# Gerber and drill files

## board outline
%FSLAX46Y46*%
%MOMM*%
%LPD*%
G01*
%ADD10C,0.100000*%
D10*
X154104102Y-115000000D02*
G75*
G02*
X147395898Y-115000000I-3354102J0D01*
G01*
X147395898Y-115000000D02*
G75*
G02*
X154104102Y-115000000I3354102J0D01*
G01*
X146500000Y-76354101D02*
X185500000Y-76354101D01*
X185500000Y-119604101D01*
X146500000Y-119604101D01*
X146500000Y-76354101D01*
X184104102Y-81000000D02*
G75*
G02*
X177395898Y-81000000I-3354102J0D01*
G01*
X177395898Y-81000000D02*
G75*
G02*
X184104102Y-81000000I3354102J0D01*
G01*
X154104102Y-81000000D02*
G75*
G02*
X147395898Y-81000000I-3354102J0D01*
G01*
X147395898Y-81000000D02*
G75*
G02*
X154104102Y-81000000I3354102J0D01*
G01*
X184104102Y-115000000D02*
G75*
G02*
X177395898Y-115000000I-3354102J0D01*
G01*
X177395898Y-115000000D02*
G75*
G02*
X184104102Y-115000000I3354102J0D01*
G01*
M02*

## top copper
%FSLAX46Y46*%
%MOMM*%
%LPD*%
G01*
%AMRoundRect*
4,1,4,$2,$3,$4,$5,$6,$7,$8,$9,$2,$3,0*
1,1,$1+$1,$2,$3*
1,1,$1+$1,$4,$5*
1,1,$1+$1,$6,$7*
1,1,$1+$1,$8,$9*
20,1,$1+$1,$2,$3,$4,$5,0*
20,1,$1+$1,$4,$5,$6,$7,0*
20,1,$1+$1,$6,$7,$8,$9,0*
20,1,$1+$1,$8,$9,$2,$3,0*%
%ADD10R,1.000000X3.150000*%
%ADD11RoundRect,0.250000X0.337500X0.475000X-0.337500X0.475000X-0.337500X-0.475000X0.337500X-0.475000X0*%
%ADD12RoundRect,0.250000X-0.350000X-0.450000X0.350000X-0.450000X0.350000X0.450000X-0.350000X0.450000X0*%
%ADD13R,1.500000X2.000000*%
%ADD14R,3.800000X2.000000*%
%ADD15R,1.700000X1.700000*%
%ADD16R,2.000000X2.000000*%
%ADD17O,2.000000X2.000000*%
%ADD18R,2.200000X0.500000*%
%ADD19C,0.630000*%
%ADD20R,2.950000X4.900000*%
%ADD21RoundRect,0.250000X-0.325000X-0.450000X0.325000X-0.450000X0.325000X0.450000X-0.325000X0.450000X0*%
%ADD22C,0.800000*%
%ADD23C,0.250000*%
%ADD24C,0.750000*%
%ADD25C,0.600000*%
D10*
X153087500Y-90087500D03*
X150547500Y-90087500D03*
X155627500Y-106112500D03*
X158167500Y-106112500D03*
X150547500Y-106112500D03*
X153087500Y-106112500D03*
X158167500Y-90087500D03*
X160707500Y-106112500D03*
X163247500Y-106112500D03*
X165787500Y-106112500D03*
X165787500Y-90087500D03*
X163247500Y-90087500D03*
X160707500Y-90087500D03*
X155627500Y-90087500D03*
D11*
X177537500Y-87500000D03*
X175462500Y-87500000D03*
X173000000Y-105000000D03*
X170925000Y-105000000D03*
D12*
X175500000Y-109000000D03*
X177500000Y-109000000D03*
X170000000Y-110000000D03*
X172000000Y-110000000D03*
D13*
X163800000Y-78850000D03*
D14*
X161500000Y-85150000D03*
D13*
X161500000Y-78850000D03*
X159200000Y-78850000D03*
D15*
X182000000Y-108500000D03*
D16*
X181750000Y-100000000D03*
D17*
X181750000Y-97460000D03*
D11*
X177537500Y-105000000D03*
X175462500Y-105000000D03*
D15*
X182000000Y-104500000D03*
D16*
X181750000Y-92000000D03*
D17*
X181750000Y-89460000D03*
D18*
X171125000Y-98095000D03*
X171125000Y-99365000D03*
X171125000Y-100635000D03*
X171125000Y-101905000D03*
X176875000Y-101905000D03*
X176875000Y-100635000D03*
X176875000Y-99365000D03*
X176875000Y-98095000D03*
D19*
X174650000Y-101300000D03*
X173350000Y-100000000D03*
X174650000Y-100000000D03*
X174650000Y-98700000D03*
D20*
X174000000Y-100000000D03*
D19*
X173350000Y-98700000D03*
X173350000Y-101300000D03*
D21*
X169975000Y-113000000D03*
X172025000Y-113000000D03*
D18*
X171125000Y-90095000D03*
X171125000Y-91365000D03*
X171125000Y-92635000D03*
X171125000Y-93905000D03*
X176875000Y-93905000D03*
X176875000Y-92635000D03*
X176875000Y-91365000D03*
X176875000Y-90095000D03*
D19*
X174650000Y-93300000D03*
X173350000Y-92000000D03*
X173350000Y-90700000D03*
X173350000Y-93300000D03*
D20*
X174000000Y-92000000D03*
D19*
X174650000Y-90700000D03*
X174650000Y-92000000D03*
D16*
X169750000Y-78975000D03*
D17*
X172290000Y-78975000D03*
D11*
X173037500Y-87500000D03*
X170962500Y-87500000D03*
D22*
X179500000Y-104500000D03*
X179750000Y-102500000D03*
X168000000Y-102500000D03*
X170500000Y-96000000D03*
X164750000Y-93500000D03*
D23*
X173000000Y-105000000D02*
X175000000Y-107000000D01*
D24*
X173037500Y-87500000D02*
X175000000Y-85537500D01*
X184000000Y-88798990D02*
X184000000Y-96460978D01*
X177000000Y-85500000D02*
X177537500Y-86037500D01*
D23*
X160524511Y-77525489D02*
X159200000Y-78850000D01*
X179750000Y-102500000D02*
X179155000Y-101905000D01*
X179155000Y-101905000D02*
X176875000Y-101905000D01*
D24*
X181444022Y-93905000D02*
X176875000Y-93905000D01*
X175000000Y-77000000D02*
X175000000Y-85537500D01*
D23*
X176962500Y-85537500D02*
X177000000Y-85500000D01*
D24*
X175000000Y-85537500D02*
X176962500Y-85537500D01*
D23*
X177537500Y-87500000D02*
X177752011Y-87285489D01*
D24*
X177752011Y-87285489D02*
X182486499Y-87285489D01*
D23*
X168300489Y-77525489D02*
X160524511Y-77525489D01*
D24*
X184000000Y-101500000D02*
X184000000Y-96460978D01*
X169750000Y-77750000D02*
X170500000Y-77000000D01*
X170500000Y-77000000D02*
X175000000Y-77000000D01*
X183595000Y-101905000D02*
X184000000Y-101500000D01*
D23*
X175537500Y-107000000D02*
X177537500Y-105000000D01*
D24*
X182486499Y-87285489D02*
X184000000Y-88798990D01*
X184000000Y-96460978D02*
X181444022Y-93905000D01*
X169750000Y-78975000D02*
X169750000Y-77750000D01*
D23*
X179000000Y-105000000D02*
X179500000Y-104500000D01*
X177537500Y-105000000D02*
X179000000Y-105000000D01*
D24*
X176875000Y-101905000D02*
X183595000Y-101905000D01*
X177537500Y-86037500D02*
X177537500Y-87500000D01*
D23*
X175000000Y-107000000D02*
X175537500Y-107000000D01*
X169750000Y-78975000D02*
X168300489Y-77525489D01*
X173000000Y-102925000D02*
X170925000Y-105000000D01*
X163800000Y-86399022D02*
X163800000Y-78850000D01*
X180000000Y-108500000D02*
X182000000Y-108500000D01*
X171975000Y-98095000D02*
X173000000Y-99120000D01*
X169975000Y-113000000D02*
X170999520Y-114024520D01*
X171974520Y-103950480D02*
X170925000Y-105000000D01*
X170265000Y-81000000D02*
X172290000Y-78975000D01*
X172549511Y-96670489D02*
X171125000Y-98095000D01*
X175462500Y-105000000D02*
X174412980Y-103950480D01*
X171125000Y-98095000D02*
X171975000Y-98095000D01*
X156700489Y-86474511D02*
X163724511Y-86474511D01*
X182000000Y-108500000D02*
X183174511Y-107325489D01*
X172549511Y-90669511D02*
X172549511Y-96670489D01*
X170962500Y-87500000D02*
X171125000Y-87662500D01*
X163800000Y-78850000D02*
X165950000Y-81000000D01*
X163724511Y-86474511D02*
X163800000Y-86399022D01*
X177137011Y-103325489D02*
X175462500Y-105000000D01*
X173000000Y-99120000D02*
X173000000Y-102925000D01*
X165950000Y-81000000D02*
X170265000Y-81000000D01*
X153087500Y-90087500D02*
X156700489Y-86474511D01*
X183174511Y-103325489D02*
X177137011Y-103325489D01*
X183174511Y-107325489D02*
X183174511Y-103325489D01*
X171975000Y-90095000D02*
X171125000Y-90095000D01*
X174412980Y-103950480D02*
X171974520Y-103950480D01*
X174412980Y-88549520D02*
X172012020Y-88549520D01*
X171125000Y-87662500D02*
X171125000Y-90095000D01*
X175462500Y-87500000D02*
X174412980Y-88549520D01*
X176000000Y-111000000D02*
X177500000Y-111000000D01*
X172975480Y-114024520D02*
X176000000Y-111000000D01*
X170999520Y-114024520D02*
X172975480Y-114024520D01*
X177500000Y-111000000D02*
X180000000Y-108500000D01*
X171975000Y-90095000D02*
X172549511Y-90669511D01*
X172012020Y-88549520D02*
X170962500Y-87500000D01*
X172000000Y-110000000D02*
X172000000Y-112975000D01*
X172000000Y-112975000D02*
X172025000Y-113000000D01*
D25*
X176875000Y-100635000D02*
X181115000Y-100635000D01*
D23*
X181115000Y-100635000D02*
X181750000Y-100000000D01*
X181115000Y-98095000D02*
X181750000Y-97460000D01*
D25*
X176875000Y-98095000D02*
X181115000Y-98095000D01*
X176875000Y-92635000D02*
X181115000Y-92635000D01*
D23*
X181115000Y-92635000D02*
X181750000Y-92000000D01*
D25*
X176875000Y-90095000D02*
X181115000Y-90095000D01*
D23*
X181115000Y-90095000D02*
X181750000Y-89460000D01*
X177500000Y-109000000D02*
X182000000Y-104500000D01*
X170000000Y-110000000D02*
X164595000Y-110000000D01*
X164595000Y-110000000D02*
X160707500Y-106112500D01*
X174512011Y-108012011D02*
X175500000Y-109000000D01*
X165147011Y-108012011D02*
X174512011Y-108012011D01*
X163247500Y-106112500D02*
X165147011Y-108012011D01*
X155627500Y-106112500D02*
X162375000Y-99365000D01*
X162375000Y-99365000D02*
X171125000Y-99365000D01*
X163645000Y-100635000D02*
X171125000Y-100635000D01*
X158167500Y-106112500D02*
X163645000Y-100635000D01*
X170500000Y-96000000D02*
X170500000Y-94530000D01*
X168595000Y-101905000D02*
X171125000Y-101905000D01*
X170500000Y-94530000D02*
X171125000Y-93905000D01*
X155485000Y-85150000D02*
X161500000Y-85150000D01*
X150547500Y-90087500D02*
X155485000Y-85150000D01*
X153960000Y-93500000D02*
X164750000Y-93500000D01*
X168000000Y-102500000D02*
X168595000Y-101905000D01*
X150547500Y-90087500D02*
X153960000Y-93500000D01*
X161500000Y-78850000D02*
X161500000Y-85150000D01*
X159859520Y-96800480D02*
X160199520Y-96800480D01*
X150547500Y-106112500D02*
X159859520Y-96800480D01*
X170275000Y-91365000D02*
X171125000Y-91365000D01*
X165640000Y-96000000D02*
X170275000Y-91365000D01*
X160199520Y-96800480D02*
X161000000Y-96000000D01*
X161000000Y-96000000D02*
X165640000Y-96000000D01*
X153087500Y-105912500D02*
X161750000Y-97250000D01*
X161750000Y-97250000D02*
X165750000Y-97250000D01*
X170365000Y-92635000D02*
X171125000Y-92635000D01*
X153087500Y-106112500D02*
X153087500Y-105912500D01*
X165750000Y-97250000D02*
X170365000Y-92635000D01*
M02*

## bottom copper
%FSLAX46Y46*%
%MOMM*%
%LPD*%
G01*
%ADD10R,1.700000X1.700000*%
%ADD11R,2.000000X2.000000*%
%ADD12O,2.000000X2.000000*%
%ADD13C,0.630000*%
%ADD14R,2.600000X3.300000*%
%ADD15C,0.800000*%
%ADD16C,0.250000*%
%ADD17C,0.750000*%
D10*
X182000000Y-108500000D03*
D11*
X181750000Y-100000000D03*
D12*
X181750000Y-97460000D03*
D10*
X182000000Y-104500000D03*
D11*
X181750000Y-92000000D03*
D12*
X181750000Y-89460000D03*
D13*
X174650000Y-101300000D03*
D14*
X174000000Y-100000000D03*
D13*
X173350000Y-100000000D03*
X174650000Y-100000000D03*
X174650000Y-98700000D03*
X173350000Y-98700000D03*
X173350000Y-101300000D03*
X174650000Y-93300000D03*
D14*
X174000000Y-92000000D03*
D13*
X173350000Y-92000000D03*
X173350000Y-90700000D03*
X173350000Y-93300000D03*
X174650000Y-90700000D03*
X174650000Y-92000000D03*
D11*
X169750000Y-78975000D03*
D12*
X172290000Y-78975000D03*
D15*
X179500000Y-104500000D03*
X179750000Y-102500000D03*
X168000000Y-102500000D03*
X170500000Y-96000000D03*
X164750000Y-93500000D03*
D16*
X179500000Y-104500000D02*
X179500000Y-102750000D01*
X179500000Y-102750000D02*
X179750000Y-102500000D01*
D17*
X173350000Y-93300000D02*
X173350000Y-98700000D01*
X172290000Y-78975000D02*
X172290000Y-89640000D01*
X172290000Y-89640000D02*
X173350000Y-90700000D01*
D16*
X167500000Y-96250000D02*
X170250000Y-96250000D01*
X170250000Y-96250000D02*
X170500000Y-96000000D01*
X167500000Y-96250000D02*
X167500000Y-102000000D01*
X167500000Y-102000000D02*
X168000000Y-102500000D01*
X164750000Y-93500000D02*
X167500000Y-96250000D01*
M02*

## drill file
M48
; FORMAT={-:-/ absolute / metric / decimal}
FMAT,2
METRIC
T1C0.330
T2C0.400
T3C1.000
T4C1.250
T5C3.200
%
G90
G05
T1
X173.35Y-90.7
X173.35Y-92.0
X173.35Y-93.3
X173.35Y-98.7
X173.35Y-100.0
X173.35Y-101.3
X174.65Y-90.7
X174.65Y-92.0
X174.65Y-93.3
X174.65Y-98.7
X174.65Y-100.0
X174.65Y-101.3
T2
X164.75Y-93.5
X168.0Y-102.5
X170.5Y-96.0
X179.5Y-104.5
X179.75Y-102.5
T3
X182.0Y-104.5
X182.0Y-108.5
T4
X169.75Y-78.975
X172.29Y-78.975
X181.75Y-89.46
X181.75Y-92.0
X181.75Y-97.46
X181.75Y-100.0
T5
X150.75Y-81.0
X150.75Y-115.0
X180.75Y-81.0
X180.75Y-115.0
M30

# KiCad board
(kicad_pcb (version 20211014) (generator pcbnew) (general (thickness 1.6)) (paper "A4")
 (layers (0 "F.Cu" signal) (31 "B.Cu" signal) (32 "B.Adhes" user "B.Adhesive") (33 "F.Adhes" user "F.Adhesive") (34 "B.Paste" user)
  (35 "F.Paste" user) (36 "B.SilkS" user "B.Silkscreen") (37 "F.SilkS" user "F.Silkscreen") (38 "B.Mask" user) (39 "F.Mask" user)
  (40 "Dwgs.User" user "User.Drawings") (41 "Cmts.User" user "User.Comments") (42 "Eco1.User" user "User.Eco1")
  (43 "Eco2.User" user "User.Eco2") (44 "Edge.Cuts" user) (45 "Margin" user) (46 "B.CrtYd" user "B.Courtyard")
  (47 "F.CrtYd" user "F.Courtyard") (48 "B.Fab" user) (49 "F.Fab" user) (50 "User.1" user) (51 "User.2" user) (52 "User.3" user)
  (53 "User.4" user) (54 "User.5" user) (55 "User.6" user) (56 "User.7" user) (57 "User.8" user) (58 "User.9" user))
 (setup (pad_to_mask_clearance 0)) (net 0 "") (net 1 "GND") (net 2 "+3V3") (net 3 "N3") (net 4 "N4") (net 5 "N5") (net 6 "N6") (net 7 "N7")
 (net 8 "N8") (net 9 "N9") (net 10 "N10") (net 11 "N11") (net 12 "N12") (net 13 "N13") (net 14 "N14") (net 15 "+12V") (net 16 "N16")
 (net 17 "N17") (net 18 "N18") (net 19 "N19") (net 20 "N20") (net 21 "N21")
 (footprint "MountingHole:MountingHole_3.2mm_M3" (layer "F.Cu") (at 180.75 115)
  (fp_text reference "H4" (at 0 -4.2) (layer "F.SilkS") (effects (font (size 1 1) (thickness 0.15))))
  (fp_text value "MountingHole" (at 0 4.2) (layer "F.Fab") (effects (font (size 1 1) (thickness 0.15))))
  (pad "" np_thru_hole circle (at 0 0) (size 3.2 3.2) (drill 3.2) (layers *.Cu *.Mask)))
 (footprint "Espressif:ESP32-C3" (layer "F.Cu") (at 159.9675 97.5125 90)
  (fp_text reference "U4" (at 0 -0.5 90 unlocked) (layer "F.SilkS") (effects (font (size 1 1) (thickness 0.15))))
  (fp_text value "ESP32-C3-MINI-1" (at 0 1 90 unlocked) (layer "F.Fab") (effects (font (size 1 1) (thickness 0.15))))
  (pad "1" smd rect (at 7.425 -6.88 90) (size 3.15 1) (layers "F.Cu" "F.Paste" "F.Mask") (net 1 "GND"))
  (pad "3" smd rect (at 7.425 -9.42 90) (size 3.15 1) (layers "F.Cu" "F.Paste" "F.Mask") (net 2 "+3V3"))
  (pad "5" smd rect (at -8.6 -4.34 90) (size 3.15 1) (layers "F.Cu" "F.Paste" "F.Mask") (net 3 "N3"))
  (pad "6" smd rect (at -8.6 -1.8 90) (size 3.15 1) (layers "F.Cu" "F.Paste" "F.Mask") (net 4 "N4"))
  (pad "12" smd rect (at -8.6 -9.42 90) (size 3.15 1) (layers "F.Cu" "F.Paste" "F.Mask") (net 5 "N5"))
  (pad "13" smd rect (at -8.6 -6.88 90) (size 3.15 1) (layers "F.Cu" "F.Paste" "F.Mask") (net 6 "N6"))
  (pad "16" smd rect (at 7.425 -1.8 90) (size 3.15 1) (layers "F.Cu" "F.Paste" "F.Mask") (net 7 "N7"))
  (pad "18" smd rect (at -8.6 0.74 90) (size 3.15 1) (layers "F.Cu" "F.Paste" "F.Mask") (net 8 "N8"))
  (pad "19" smd rect (at -8.6 3.28 90) (size 3.15 1) (layers "F.Cu" "F.Paste" "F.Mask") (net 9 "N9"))
  (pad "20" smd rect (at -8.6 5.82 90) (size 3.15 1) (layers "F.Cu" "F.Paste" "F.Mask") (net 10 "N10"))
  (pad "21" smd rect (at 7.425 5.82 90) (size 3.15 1) (layers "F.Cu" "F.Paste" "F.Mask") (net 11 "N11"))
  (pad "22" smd rect (at 7.425 3.28 90) (size 3.15 1) (layers "F.Cu" "F.Paste" "F.Mask") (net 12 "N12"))
  (pad "23" smd rect (at 7.425 0.74 90) (size 3.15 1) (layers "F.Cu" "F.Paste" "F.Mask") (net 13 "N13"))
  (pad "35" smd rect (at 7.425 -4.34 90) (size 3.15 1) (layers "F.Cu" "F.Paste" "F.Mask") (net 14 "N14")))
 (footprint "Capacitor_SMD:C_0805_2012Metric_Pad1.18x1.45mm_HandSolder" (layer "F.Cu") (at 176.5 87.5 180)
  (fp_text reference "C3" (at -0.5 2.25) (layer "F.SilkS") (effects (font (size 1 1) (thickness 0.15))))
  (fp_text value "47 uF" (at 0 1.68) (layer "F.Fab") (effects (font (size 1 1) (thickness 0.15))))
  (pad "1" smd roundrect (at -1.0375 0 180) (size 1.175 1.45) (layers "F.Cu" "F.Paste" "F.Mask") (roundrect_rratio 0.2127659574)
   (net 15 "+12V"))
  (pad "2" smd roundrect (at 1.0375 0 180) (size 1.175 1.45) (layers "F.Cu" "F.Paste" "F.Mask") (roundrect_rratio 0.2127659574)
   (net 1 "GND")))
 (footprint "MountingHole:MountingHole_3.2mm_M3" (layer "F.Cu") (at 180.75 81)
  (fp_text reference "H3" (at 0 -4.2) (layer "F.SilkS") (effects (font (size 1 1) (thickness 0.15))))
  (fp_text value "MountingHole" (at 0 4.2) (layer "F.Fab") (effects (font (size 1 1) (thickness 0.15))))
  (pad "" np_thru_hole circle (at 0 0) (size 3.2 3.2) (drill 3.2) (layers *.Cu *.Mask)))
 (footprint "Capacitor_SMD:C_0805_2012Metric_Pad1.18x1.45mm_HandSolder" (layer "F.Cu") (at 171.9625 105 180)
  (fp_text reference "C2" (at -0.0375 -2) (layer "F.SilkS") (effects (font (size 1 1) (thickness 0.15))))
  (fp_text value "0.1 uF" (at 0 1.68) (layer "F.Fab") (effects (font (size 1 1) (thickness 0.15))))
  (pad "1" smd roundrect (at -1.0375 0 180) (size 1.175 1.45) (layers "F.Cu" "F.Paste" "F.Mask") (roundrect_rratio 0.2127659574)
   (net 15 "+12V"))
  (pad "2" smd roundrect (at 1.0375 0 180) (size 1.175 1.45) (layers "F.Cu" "F.Paste" "F.Mask") (roundrect_rratio 0.2127659574)
   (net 1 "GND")))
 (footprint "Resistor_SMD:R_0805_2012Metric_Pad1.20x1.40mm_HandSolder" (layer "F.Cu") (at 176.5 109)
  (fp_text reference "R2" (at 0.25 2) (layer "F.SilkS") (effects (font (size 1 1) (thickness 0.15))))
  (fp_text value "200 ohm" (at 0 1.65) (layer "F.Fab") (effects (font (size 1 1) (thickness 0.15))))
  (pad "1" smd roundrect (at -1 0) (size 1.2 1.4) (layers "F.Cu" "F.Paste" "F.Mask") (roundrect_rratio 0.2083333333) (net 9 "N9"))
  (pad "2" smd roundrect (at 1 0) (size 1.2 1.4) (layers "F.Cu" "F.Paste" "F.Mask") (roundrect_rratio 0.2083333333) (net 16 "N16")))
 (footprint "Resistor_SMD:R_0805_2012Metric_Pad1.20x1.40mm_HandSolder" (layer "F.Cu") (at 171 110)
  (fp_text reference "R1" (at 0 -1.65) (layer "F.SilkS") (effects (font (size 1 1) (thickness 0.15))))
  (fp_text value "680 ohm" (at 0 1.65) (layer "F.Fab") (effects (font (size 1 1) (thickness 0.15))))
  (pad "1" smd roundrect (at -1 0) (size 1.2 1.4) (layers "F.Cu" "F.Paste" "F.Mask") (roundrect_rratio 0.2083333333) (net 8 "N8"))
  (pad "2" smd roundrect (at 1 0) (size 1.2 1.4) (layers "F.Cu" "F.Paste" "F.Mask") (roundrect_rratio 0.2083333333) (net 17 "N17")))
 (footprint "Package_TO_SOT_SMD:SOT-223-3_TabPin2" (layer "F.Cu") (at 161.5 82 -90)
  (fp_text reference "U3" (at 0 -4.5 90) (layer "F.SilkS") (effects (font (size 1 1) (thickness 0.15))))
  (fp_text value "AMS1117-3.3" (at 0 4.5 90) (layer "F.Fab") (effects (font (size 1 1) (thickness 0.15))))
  (pad "1" smd rect (at -3.15 -2.3 270) (size 2 1.5) (layers "F.Cu" "F.Paste" "F.Mask") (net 1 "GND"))
  (pad "2" smd rect (at 3.15 0 270) (size 2 3.8) (layers "F.Cu" "F.Paste" "F.Mask") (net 2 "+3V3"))
  (pad "2" smd rect (at -3.15 0 270) (size 2 1.5) (layers "F.Cu" "F.Paste" "F.Mask") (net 2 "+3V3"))
  (pad "3" smd rect (at -3.15 2.3 270) (size 2 1.5) (layers "F.Cu" "F.Paste" "F.Mask") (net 15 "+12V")))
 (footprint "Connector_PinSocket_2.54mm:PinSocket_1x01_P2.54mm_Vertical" (layer "F.Cu") (at 182 108.5 180)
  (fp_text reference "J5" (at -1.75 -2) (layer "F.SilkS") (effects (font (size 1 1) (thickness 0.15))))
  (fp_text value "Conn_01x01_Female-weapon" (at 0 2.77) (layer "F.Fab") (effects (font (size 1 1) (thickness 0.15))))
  (pad "1" thru_hole rect (at 0 0 180) (size 1.7 1.7) (drill 1) (layers *.Cu *.Mask) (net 1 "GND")))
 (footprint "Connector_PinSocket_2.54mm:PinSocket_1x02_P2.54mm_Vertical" (layer "F.Cu") (at 181.75 100 180)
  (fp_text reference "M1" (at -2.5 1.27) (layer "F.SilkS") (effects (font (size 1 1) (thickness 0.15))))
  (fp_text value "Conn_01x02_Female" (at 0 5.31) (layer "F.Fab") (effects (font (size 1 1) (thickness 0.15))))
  (pad "1" thru_hole rect (at 0 0 180) (size 2 2) (drill 1.25) (layers *.Cu *.Mask) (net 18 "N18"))
  (pad "2" thru_hole oval (at 0 2.54 180) (size 2 2) (drill 1.25) (layers *.Cu *.Mask) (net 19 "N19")))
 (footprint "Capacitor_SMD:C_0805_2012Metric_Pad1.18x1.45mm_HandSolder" (layer "F.Cu") (at 176.5 105 180)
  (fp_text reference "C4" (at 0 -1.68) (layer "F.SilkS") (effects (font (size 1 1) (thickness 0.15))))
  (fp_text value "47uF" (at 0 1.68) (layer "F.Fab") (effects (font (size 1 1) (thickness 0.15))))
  (pad "1" smd roundrect (at -1.0375 0 180) (size 1.175 1.45) (layers "F.Cu" "F.Paste" "F.Mask") (roundrect_rratio 0.2127659574)
   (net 15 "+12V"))
  (pad "2" smd roundrect (at 1.0375 0 180) (size 1.175 1.45) (layers "F.Cu" "F.Paste" "F.Mask") (roundrect_rratio 0.2127659574)
   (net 1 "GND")))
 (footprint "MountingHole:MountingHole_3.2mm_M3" (layer "F.Cu") (at 150.75 115)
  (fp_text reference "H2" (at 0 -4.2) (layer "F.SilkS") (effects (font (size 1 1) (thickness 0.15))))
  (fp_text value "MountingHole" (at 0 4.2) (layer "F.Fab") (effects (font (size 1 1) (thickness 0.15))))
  (pad "" np_thru_hole circle (at 0 0) (size 3.2 3.2) (drill 3.2) (layers *.Cu *.Mask)))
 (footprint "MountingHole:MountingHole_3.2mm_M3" (layer "F.Cu") (at 150.75 81)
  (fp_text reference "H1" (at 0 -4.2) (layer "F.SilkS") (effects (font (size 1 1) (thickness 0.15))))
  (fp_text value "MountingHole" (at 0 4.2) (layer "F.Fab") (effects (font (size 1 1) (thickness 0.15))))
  (pad "" np_thru_hole circle (at 0 0) (size 3.2 3.2) (drill 3.2) (layers *.Cu *.Mask)))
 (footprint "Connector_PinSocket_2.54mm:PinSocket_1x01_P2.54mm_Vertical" (layer "F.Cu") (at 182 104.5)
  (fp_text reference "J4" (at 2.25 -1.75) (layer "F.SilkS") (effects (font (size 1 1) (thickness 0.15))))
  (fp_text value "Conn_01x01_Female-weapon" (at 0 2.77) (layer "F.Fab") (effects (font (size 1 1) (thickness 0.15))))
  (pad "1" thru_hole rect (at 0 0) (size 1.7 1.7) (drill 1) (layers *.Cu *.Mask) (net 16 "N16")))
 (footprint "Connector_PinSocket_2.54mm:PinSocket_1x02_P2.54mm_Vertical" (layer "F.Cu") (at 181.75 92 180)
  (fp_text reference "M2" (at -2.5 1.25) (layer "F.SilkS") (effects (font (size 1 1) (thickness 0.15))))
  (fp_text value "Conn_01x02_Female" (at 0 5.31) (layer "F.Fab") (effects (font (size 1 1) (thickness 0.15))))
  (pad "1" thru_hole rect (at 0 0 180) (size 2 2) (drill 1.25) (layers *.Cu *.Mask) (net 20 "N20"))
  (pad "2" thru_hole oval (at 0 2.54 180) (size 2 2) (drill 1.25) (layers *.Cu *.Mask) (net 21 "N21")))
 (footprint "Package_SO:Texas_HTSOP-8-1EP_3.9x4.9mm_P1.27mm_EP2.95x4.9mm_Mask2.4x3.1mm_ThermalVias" (layer "F.Cu") (at 174 100)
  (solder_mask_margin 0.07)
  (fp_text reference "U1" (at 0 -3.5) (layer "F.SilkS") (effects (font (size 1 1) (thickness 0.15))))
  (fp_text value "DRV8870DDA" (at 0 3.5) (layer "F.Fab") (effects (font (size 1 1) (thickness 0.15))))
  (pad "" smd rect (at 0 0) (size 2.4 3.1) (layers "F.Paste")) (pad "" smd rect (at 0 0) (size 2.4 3.1) (layers "F.Mask"))
  (pad "1" smd rect (at -2.875 -1.905) (size 2.2 0.5) (layers "F.Cu" "F.Paste" "F.Mask") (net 1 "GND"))
  (pad "2" smd rect (at -2.875 -0.635) (size 2.2 0.5) (layers "F.Cu" "F.Paste" "F.Mask") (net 3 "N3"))
  (pad "3" smd rect (at -2.875 0.635) (size 2.2 0.5) (layers "F.Cu" "F.Paste" "F.Mask") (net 4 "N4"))
  (pad "4" smd rect (at -2.875 1.905) (size 2.2 0.5) (layers "F.Cu" "F.Paste" "F.Mask") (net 2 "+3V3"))
  (pad "5" smd rect (at 2.875 1.905) (size 2.2 0.5) (layers "F.Cu" "F.Paste" "F.Mask") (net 15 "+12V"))
  (pad "6" smd rect (at 2.875 0.635) (size 2.2 0.5) (layers "F.Cu" "F.Paste" "F.Mask") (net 18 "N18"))
  (pad "7" smd rect (at 2.875 -0.635) (size 2.2 0.5) (layers "F.Cu" "F.Paste" "F.Mask") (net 1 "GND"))
  (pad "8" smd rect (at 2.875 -1.905) (size 2.2 0.5) (layers "F.Cu" "F.Paste" "F.Mask") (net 19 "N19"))
  (pad "9" thru_hole circle (at 0.65 1.3) (size 0.63 0.63) (drill 0.33) (layers *.Cu *.Mask) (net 1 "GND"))
  (pad "9" smd rect (at 0 0) (size 2.6 3.3) (layers "B.Cu") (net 1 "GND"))
  (pad "9" thru_hole circle (at -0.65 0) (size 0.63 0.63) (drill 0.33) (layers *.Cu *.Mask) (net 1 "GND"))
  (pad "9" thru_hole circle (at 0.65 0) (size 0.63 0.63) (drill 0.33) (layers *.Cu *.Mask) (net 1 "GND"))
  (pad "9" thru_hole circle (at 0.65 -1.3) (size 0.63 0.63) (drill 0.33) (layers *.Cu *.Mask) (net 1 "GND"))
  (pad "9" smd rect (at 0 0) (size 2.95 4.9) (layers "F.Cu") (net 1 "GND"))
  (pad "9" thru_hole circle (at -0.65 -1.3) (size 0.63 0.63) (drill 0.33) (layers *.Cu *.Mask) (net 1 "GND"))
  (pad "9" thru_hole circle (at -0.65 1.3) (size 0.63 0.63) (drill 0.33) (layers *.Cu *.Mask) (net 1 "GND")))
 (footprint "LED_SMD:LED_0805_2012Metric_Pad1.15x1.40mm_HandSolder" (layer "F.Cu") (at 171 113)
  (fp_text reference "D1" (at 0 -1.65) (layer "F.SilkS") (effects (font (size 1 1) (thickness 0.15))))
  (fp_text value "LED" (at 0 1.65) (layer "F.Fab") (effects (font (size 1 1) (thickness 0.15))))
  (pad "1" smd roundrect (at -1.025 0) (size 1.15 1.4) (layers "F.Cu" "F.Paste" "F.Mask") (roundrect_rratio 0.2173913043) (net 1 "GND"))
  (pad "2" smd roundrect (at 1.025 0) (size 1.15 1.4) (layers "F.Cu" "F.Paste" "F.Mask") (roundrect_rratio 0.2173913043) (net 17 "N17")))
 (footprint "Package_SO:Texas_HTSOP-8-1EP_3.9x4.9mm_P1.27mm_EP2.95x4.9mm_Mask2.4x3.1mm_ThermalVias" (layer "F.Cu") (at 174 92)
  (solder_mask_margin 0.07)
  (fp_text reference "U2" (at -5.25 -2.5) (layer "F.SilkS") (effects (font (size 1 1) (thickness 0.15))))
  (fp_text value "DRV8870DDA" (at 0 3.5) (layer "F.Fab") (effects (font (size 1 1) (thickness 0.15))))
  (pad "" smd rect (at 0 0) (size 2.4 3.1) (layers "F.Mask")) (pad "" smd rect (at 0 0) (size 2.4 3.1) (layers "F.Paste"))
  (pad "1" smd rect (at -2.875 -1.905) (size 2.2 0.5) (layers "F.Cu" "F.Paste" "F.Mask") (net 1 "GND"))
  (pad "2" smd rect (at -2.875 -0.635) (size 2.2 0.5) (layers "F.Cu" "F.Paste" "F.Mask") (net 5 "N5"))
  (pad "3" smd rect (at -2.875 0.635) (size 2.2 0.5) (layers "F.Cu" "F.Paste" "F.Mask") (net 6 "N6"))
  (pad "4" smd rect (at -2.875 1.905) (size 2.2 0.5) (layers "F.Cu" "F.Paste" "F.Mask") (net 2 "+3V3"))
  (pad "5" smd rect (at 2.875 1.905) (size 2.2 0.5) (layers "F.Cu" "F.Paste" "F.Mask") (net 15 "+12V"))
  (pad "6" smd rect (at 2.875 0.635) (size 2.2 0.5) (layers "F.Cu" "F.Paste" "F.Mask") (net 20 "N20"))
  (pad "7" smd rect (at 2.875 -0.635) (size 2.2 0.5) (layers "F.Cu" "F.Paste" "F.Mask") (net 1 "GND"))
  (pad "8" smd rect (at 2.875 -1.905) (size 2.2 0.5) (layers "F.Cu" "F.Paste" "F.Mask") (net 21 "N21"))
  (pad "9" thru_hole circle (at 0.65 1.3) (size 0.63 0.63) (drill 0.33) (layers *.Cu *.Mask) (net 1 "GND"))
  (pad "9" smd rect (at 0 0) (size 2.6 3.3) (layers "B.Cu") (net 1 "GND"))
  (pad "9" thru_hole circle (at -0.65 0) (size 0.63 0.63) (drill 0.33) (layers *.Cu *.Mask) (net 1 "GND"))
  (pad "9" thru_hole circle (at -0.65 -1.3) (size 0.63 0.63) (drill 0.33) (layers *.Cu *.Mask) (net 1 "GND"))
  (pad "9" thru_hole circle (at -0.65 1.3) (size 0.63 0.63) (drill 0.33) (layers *.Cu *.Mask) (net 1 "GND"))
  (pad "9" smd rect (at 0 0) (size 2.95 4.9) (layers "F.Cu") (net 1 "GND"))
  (pad "9" thru_hole circle (at 0.65 -1.3) (size 0.63 0.63) (drill 0.33) (layers *.Cu *.Mask) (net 1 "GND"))
  (pad "9" thru_hole circle (at 0.65 0) (size 0.63 0.63) (drill 0.33) (layers *.Cu *.Mask) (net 1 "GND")))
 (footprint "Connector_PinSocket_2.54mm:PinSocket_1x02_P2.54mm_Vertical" (layer "F.Cu") (at 169.75 78.975 90)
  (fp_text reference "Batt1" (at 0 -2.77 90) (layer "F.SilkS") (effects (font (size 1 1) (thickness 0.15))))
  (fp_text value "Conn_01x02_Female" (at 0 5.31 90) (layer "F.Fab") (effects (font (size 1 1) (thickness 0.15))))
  (pad "1" thru_hole rect (at 0 0 90) (size 2 2) (drill 1.25) (layers *.Cu *.Mask) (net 15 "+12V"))
  (pad "2" thru_hole oval (at 0 2.54 90) (size 2 2) (drill 1.25) (layers *.Cu *.Mask) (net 1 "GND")))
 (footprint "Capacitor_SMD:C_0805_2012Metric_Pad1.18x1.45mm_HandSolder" (layer "F.Cu") (at 172 87.5 180)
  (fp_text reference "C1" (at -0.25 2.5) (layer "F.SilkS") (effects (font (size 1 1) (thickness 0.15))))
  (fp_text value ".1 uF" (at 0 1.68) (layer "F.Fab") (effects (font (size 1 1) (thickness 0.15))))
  (pad "1" smd roundrect (at -1.0375 0 180) (size 1.175 1.45) (layers "F.Cu" "F.Paste" "F.Mask") (roundrect_rratio 0.2127659574)
   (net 15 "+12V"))
  (pad "2" smd roundrect (at 1.0375 0 180) (size 1.175 1.45) (layers "F.Cu" "F.Paste" "F.Mask") (roundrect_rratio 0.2127659574)
   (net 1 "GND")))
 (gr_circle (center 150.75 115) (end 153.75 116.5) (layer "Edge.Cuts") (width 0.1) (fill none))
 (gr_rect (start 146.5 76.354101) (end 185.5 119.604101) (layer "Edge.Cuts") (width 0.1) (fill none))
 (gr_circle (center 180.75 81) (end 183.75 82.5) (layer "Edge.Cuts") (width 0.1) (fill none))
 (gr_circle (center 150.75 81) (end 153.75 82.5) (layer "Edge.Cuts") (width 0.1) (fill none))
 (gr_circle (center 180.75 115) (end 183.75 116.5) (layer "Edge.Cuts") (width 0.1) (fill none))
 (segment (start 173 105) (end 175 107) (width 0.25) (layer "F.Cu") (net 15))
 (segment (start 173.0375 87.5) (end 175 85.5375) (width 0.75) (layer "F.Cu") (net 15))
 (segment (start 184 88.79899) (end 184 96.460978) (width 0.75) (layer "F.Cu") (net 15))
 (segment (start 177 85.5) (end 177.5375 86.0375) (width 0.75) (layer "F.Cu") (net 15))
 (segment (start 160.524511 77.525489) (end 159.2 78.85) (width 0.25) (layer "F.Cu") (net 15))
 (segment (start 179.75 102.5) (end 179.155 101.905) (width 0.25) (layer "F.Cu") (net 15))
 (segment (start 179.155 101.905) (end 176.875 101.905) (width 0.25) (layer "F.Cu") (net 15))
 (segment (start 181.444022 93.905) (end 176.875 93.905) (width 0.75) (layer "F.Cu") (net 15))
 (segment (start 175 77) (end 175 85.5375) (width 0.75) (layer "F.Cu") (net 15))
 (segment (start 176.9625 85.5375) (end 177 85.5) (width 0.25) (layer "F.Cu") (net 15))
 (segment (start 175 85.5375) (end 176.9625 85.5375) (width 0.75) (layer "F.Cu") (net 15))
 (segment (start 177.5375 87.5) (end 177.752011 87.285489) (width 0.25) (layer "F.Cu") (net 15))
 (segment (start 177.752011 87.285489) (end 182.486499 87.285489) (width 0.75) (layer "F.Cu") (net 15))
 (segment (start 168.300489 77.525489) (end 160.524511 77.525489) (width 0.25) (layer "F.Cu") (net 15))
 (segment (start 184 101.5) (end 184 96.460978) (width 0.75) (layer "F.Cu") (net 15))
 (segment (start 169.75 77.75) (end 170.5 77) (width 0.75) (layer "F.Cu") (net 15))
 (segment (start 170.5 77) (end 175 77) (width 0.75) (layer "F.Cu") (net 15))
 (segment (start 183.595 101.905) (end 184 101.5) (width 0.75) (layer "F.Cu") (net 15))
 (segment (start 175.5375 107) (end 177.5375 105) (width 0.25) (layer "F.Cu") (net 15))
 (segment (start 182.486499 87.285489) (end 184 88.79899) (width 0.75) (layer "F.Cu") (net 15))
 (segment (start 184 96.460978) (end 181.444022 93.905) (width 0.75) (layer "F.Cu") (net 15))
 (segment (start 169.75 78.975) (end 169.75 77.75) (width 0.75) (layer "F.Cu") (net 15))
 (segment (start 179 105) (end 179.5 104.5) (width 0.25) (layer "F.Cu") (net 15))
 (segment (start 177.5375 105) (end 179 105) (width 0.25) (layer "F.Cu") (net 15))
 (segment (start 176.875 101.905) (end 183.595 101.905) (width 0.75) (layer "F.Cu") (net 15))
 (segment (start 177.5375 86.0375) (end 177.5375 87.5) (width 0.75) (layer "F.Cu") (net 15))
 (segment (start 175 107) (end 175.5375 107) (width 0.25) (layer "F.Cu") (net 15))
 (segment (start 169.75 78.975) (end 168.300489 77.525489) (width 0.25) (layer "F.Cu") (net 15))
 (via (at 179.5 104.5) (size 0.8) (drill 0.4) (layers "F.Cu" "B.Cu") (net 15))
 (via (at 179.75 102.5) (size 0.8) (drill 0.4) (layers "F.Cu" "B.Cu") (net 15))
 (segment (start 179.5 104.5) (end 179.5 102.75) (width 0.25) (layer "B.Cu") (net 15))
 (segment (start 179.5 102.75) (end 179.75 102.5) (width 0.25) (layer "B.Cu") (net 15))
 (segment (start 173 102.925) (end 170.925 105) (width 0.25) (layer "F.Cu") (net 1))
 (segment (start 163.8 86.399022) (end 163.8 78.85) (width 0.25) (layer "F.Cu") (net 1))
 (segment (start 180 108.5) (end 182 108.5) (width 0.25) (layer "F.Cu") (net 1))
 (segment (start 171.975 98.095) (end 173 99.12) (width 0.25) (layer "F.Cu") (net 1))
 (segment (start 169.975 113) (end 170.99952 114.02452) (width 0.25) (layer "F.Cu") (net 1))
 (segment (start 171.97452 103.95048) (end 170.925 105) (width 0.25) (layer "F.Cu") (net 1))
 (segment (start 170.265 81) (end 172.29 78.975) (width 0.25) (layer "F.Cu") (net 1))
 (segment (start 172.549511 96.670489) (end 171.125 98.095) (width 0.25) (layer "F.Cu") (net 1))
 (segment (start 175.4625 105) (end 174.41298 103.95048) (width 0.25) (layer "F.Cu") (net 1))
 (segment (start 171.125 98.095) (end 171.975 98.095) (width 0.25) (layer "F.Cu") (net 1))
 (segment (start 156.700489 86.474511) (end 163.724511 86.474511) (width 0.25) (layer "F.Cu") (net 1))
 (segment (start 182 108.5) (end 183.174511 107.325489) (width 0.25) (layer "F.Cu") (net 1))
 (segment (start 172.549511 90.669511) (end 172.549511 96.670489) (width 0.25) (layer "F.Cu") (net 1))
 (segment (start 170.9625 87.5) (end 171.125 87.6625) (width 0.25) (layer "F.Cu") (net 1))
 (segment (start 163.8 78.85) (end 165.95 81) (width 0.25) (layer "F.Cu") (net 1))
 (segment (start 163.724511 86.474511) (end 163.8 86.399022) (width 0.25) (layer "F.Cu") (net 1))
 (segment (start 177.137011 103.325489) (end 175.4625 105) (width 0.25) (layer "F.Cu") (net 1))
 (segment (start 173 99.12) (end 173 102.925) (width 0.25) (layer "F.Cu") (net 1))
 (segment (start 165.95 81) (end 170.265 81) (width 0.25) (layer "F.Cu") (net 1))
 (segment (start 153.0875 90.0875) (end 156.700489 86.474511) (width 0.25) (layer "F.Cu") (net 1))
 (segment (start 183.174511 103.325489) (end 177.137011 103.325489) (width 0.25) (layer "F.Cu") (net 1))
 (segment (start 183.174511 107.325489) (end 183.174511 103.325489) (width 0.25) (layer "F.Cu") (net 1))
 (segment (start 171.975 90.095) (end 171.125 90.095) (width 0.25) (layer "F.Cu") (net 1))
 (segment (start 174.41298 103.95048) (end 171.97452 103.95048) (width 0.25) (layer "F.Cu") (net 1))
 (segment (start 174.41298 88.54952) (end 172.01202 88.54952) (width 0.25) (layer "F.Cu") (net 1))
 (segment (start 171.125 87.6625) (end 171.125 90.095) (width 0.25) (layer "F.Cu") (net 1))
 (segment (start 175.4625 87.5) (end 174.41298 88.54952) (width 0.25) (layer "F.Cu") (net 1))
 (segment (start 176 111) (end 177.5 111) (width 0.25) (layer "F.Cu") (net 1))
 (segment (start 172.97548 114.02452) (end 176 111) (width 0.25) (layer "F.Cu") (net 1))
 (segment (start 170.99952 114.02452) (end 172.97548 114.02452) (width 0.25) (layer "F.Cu") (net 1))
 (segment (start 177.5 111) (end 180 108.5) (width 0.25) (layer "F.Cu") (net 1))
 (segment (start 171.975 90.095) (end 172.549511 90.669511) (width 0.25) (layer "F.Cu") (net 1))
 (segment (start 172.01202 88.54952) (end 170.9625 87.5) (width 0.25) (layer "F.Cu") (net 1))
 (segment (start 173.35 93.3) (end 173.35 98.7) (width 0.75) (layer "B.Cu") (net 1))
 (segment (start 172.29 78.975) (end 172.29 89.64) (width 0.75) (layer "B.Cu") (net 1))
 (segment (start 172.29 89.64) (end 173.35 90.7) (width 0.75) (layer "B.Cu") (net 1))
 (segment (start 172 110) (end 172 112.975) (width 0.25) (layer "F.Cu") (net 17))
 (segment (start 172 112.975) (end 172.025 113) (width 0.25) (layer "F.Cu") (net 17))
 (segment (start 176.875 100.635) (end 181.115 100.635) (width 0.6) (layer "F.Cu") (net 18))
 (segment (start 181.115 100.635) (end 181.75 100) (width 0.25) (layer "F.Cu") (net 18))
 (segment (start 181.115 98.095) (end 181.75 97.46) (width 0.25) (layer "F.Cu") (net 19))
 (segment (start 176.875 98.095) (end 181.115 98.095) (width 0.6) (layer "F.Cu") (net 19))
 (segment (start 176.875 92.635) (end 181.115 92.635) (width 0.6) (layer "F.Cu") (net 20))
 (segment (start 181.115 92.635) (end 181.75 92) (width 0.25) (layer "F.Cu") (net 20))
 (segment (start 176.875 90.095) (end 181.115 90.095) (width 0.6) (layer "F.Cu") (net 21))
 (segment (start 181.115 90.095) (end 181.75 89.46) (width 0.25) (layer "F.Cu") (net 21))
 (segment (start 177.5 109) (end 182 104.5) (width 0.25) (layer "F.Cu") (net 16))
 (segment (start 170 110) (end 164.595 110) (width 0.25) (layer "F.Cu") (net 8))
 (segment (start 164.595 110) (end 160.7075 106.1125) (width 0.25) (layer "F.Cu") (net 8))
 (segment (start 174.512011 108.012011) (end 175.5 109) (width 0.25) (layer "F.Cu") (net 9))
 (segment (start 165.147011 108.012011) (end 174.512011 108.012011) (width 0.25) (layer "F.Cu") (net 9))
 (segment (start 163.2475 106.1125) (end 165.147011 108.012011) (width 0.25) (layer "F.Cu") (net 9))
 (segment (start 155.6275 106.1125) (end 162.375 99.365) (width 0.25) (layer "F.Cu") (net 3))
 (segment (start 162.375 99.365) (end 171.125 99.365) (width 0.25) (layer "F.Cu") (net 3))
 (segment (start 163.645 100.635) (end 171.125 100.635) (width 0.25) (layer "F.Cu") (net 4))
 (segment (start 158.1675 106.1125) (end 163.645 100.635) (width 0.25) (layer "F.Cu") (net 4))
 (segment (start 170.5 96) (end 170.5 94.53) (width 0.25) (layer "F.Cu") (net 2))
 (segment (start 168.595 101.905) (end 171.125 101.905) (width 0.25) (layer "F.Cu") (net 2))
 (segment (start 170.5 94.53) (end 171.125 93.905) (width 0.25) (layer "F.Cu") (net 2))
 (segment (start 155.485 85.15) (end 161.5 85.15) (width 0.25) (layer "F.Cu") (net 2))
 (segment (start 150.5475 90.0875) (end 155.485 85.15) (width 0.25) (layer "F.Cu") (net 2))
 (segment (start 153.96 93.5) (end 164.75 93.5) (width 0.25) (layer "F.Cu") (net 2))
 (segment (start 168 102.5) (end 168.595 101.905) (width 0.25) (layer "F.Cu") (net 2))
 (segment (start 150.5475 90.0875) (end 153.96 93.5) (width 0.25) (layer "F.Cu") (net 2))
 (segment (start 161.5 78.85) (end 161.5 85.15) (width 0.25) (layer "F.Cu") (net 2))
 (via (at 168 102.5) (size 0.8) (drill 0.4) (layers "F.Cu" "B.Cu") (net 2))
 (via (at 170.5 96) (size 0.8) (drill 0.4) (layers "F.Cu" "B.Cu") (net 2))
 (via (at 164.75 93.5) (size 0.8) (drill 0.4) (layers "F.Cu" "B.Cu") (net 2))
 (segment (start 167.5 96.25) (end 170.25 96.25) (width 0.25) (layer "B.Cu") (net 2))
 (segment (start 170.25 96.25) (end 170.5 96) (width 0.25) (layer "B.Cu") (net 2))
 (segment (start 167.5 96.25) (end 167.5 102) (width 0.25) (layer "B.Cu") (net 2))
 (segment (start 167.5 102) (end 168 102.5) (width 0.25) (layer "B.Cu") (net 2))
 (segment (start 164.75 93.5) (end 167.5 96.25) (width 0.25) (layer "B.Cu") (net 2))
 (segment (start 159.85952 96.80048) (end 160.19952 96.80048) (width 0.25) (layer "F.Cu") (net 5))
 (segment (start 150.5475 106.1125) (end 159.85952 96.80048) (width 0.25) (layer "F.Cu") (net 5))
 (segment (start 170.275 91.365) (end 171.125 91.365) (width 0.25) (layer "F.Cu") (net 5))
 (segment (start 165.64 96) (end 170.275 91.365) (width 0.25) (layer "F.Cu") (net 5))
 (segment (start 160.19952 96.80048) (end 161 96) (width 0.25) (layer "F.Cu") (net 5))
 (segment (start 161 96) (end 165.64 96) (width 0.25) (layer "F.Cu") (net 5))
 (segment (start 153.0875 105.9125) (end 161.75 97.25) (width 0.25) (layer "F.Cu") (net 6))
 (segment (start 161.75 97.25) (end 165.75 97.25) (width 0.25) (layer "F.Cu") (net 6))
 (segment (start 170.365 92.635) (end 171.125 92.635) (width 0.25) (layer "F.Cu") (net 6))
 (segment (start 153.0875 106.1125) (end 153.0875 105.9125) (width 0.25) (layer "F.Cu") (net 6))
 (segment (start 165.75 97.25) (end 170.365 92.635) (width 0.25) (layer "F.Cu") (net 6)))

